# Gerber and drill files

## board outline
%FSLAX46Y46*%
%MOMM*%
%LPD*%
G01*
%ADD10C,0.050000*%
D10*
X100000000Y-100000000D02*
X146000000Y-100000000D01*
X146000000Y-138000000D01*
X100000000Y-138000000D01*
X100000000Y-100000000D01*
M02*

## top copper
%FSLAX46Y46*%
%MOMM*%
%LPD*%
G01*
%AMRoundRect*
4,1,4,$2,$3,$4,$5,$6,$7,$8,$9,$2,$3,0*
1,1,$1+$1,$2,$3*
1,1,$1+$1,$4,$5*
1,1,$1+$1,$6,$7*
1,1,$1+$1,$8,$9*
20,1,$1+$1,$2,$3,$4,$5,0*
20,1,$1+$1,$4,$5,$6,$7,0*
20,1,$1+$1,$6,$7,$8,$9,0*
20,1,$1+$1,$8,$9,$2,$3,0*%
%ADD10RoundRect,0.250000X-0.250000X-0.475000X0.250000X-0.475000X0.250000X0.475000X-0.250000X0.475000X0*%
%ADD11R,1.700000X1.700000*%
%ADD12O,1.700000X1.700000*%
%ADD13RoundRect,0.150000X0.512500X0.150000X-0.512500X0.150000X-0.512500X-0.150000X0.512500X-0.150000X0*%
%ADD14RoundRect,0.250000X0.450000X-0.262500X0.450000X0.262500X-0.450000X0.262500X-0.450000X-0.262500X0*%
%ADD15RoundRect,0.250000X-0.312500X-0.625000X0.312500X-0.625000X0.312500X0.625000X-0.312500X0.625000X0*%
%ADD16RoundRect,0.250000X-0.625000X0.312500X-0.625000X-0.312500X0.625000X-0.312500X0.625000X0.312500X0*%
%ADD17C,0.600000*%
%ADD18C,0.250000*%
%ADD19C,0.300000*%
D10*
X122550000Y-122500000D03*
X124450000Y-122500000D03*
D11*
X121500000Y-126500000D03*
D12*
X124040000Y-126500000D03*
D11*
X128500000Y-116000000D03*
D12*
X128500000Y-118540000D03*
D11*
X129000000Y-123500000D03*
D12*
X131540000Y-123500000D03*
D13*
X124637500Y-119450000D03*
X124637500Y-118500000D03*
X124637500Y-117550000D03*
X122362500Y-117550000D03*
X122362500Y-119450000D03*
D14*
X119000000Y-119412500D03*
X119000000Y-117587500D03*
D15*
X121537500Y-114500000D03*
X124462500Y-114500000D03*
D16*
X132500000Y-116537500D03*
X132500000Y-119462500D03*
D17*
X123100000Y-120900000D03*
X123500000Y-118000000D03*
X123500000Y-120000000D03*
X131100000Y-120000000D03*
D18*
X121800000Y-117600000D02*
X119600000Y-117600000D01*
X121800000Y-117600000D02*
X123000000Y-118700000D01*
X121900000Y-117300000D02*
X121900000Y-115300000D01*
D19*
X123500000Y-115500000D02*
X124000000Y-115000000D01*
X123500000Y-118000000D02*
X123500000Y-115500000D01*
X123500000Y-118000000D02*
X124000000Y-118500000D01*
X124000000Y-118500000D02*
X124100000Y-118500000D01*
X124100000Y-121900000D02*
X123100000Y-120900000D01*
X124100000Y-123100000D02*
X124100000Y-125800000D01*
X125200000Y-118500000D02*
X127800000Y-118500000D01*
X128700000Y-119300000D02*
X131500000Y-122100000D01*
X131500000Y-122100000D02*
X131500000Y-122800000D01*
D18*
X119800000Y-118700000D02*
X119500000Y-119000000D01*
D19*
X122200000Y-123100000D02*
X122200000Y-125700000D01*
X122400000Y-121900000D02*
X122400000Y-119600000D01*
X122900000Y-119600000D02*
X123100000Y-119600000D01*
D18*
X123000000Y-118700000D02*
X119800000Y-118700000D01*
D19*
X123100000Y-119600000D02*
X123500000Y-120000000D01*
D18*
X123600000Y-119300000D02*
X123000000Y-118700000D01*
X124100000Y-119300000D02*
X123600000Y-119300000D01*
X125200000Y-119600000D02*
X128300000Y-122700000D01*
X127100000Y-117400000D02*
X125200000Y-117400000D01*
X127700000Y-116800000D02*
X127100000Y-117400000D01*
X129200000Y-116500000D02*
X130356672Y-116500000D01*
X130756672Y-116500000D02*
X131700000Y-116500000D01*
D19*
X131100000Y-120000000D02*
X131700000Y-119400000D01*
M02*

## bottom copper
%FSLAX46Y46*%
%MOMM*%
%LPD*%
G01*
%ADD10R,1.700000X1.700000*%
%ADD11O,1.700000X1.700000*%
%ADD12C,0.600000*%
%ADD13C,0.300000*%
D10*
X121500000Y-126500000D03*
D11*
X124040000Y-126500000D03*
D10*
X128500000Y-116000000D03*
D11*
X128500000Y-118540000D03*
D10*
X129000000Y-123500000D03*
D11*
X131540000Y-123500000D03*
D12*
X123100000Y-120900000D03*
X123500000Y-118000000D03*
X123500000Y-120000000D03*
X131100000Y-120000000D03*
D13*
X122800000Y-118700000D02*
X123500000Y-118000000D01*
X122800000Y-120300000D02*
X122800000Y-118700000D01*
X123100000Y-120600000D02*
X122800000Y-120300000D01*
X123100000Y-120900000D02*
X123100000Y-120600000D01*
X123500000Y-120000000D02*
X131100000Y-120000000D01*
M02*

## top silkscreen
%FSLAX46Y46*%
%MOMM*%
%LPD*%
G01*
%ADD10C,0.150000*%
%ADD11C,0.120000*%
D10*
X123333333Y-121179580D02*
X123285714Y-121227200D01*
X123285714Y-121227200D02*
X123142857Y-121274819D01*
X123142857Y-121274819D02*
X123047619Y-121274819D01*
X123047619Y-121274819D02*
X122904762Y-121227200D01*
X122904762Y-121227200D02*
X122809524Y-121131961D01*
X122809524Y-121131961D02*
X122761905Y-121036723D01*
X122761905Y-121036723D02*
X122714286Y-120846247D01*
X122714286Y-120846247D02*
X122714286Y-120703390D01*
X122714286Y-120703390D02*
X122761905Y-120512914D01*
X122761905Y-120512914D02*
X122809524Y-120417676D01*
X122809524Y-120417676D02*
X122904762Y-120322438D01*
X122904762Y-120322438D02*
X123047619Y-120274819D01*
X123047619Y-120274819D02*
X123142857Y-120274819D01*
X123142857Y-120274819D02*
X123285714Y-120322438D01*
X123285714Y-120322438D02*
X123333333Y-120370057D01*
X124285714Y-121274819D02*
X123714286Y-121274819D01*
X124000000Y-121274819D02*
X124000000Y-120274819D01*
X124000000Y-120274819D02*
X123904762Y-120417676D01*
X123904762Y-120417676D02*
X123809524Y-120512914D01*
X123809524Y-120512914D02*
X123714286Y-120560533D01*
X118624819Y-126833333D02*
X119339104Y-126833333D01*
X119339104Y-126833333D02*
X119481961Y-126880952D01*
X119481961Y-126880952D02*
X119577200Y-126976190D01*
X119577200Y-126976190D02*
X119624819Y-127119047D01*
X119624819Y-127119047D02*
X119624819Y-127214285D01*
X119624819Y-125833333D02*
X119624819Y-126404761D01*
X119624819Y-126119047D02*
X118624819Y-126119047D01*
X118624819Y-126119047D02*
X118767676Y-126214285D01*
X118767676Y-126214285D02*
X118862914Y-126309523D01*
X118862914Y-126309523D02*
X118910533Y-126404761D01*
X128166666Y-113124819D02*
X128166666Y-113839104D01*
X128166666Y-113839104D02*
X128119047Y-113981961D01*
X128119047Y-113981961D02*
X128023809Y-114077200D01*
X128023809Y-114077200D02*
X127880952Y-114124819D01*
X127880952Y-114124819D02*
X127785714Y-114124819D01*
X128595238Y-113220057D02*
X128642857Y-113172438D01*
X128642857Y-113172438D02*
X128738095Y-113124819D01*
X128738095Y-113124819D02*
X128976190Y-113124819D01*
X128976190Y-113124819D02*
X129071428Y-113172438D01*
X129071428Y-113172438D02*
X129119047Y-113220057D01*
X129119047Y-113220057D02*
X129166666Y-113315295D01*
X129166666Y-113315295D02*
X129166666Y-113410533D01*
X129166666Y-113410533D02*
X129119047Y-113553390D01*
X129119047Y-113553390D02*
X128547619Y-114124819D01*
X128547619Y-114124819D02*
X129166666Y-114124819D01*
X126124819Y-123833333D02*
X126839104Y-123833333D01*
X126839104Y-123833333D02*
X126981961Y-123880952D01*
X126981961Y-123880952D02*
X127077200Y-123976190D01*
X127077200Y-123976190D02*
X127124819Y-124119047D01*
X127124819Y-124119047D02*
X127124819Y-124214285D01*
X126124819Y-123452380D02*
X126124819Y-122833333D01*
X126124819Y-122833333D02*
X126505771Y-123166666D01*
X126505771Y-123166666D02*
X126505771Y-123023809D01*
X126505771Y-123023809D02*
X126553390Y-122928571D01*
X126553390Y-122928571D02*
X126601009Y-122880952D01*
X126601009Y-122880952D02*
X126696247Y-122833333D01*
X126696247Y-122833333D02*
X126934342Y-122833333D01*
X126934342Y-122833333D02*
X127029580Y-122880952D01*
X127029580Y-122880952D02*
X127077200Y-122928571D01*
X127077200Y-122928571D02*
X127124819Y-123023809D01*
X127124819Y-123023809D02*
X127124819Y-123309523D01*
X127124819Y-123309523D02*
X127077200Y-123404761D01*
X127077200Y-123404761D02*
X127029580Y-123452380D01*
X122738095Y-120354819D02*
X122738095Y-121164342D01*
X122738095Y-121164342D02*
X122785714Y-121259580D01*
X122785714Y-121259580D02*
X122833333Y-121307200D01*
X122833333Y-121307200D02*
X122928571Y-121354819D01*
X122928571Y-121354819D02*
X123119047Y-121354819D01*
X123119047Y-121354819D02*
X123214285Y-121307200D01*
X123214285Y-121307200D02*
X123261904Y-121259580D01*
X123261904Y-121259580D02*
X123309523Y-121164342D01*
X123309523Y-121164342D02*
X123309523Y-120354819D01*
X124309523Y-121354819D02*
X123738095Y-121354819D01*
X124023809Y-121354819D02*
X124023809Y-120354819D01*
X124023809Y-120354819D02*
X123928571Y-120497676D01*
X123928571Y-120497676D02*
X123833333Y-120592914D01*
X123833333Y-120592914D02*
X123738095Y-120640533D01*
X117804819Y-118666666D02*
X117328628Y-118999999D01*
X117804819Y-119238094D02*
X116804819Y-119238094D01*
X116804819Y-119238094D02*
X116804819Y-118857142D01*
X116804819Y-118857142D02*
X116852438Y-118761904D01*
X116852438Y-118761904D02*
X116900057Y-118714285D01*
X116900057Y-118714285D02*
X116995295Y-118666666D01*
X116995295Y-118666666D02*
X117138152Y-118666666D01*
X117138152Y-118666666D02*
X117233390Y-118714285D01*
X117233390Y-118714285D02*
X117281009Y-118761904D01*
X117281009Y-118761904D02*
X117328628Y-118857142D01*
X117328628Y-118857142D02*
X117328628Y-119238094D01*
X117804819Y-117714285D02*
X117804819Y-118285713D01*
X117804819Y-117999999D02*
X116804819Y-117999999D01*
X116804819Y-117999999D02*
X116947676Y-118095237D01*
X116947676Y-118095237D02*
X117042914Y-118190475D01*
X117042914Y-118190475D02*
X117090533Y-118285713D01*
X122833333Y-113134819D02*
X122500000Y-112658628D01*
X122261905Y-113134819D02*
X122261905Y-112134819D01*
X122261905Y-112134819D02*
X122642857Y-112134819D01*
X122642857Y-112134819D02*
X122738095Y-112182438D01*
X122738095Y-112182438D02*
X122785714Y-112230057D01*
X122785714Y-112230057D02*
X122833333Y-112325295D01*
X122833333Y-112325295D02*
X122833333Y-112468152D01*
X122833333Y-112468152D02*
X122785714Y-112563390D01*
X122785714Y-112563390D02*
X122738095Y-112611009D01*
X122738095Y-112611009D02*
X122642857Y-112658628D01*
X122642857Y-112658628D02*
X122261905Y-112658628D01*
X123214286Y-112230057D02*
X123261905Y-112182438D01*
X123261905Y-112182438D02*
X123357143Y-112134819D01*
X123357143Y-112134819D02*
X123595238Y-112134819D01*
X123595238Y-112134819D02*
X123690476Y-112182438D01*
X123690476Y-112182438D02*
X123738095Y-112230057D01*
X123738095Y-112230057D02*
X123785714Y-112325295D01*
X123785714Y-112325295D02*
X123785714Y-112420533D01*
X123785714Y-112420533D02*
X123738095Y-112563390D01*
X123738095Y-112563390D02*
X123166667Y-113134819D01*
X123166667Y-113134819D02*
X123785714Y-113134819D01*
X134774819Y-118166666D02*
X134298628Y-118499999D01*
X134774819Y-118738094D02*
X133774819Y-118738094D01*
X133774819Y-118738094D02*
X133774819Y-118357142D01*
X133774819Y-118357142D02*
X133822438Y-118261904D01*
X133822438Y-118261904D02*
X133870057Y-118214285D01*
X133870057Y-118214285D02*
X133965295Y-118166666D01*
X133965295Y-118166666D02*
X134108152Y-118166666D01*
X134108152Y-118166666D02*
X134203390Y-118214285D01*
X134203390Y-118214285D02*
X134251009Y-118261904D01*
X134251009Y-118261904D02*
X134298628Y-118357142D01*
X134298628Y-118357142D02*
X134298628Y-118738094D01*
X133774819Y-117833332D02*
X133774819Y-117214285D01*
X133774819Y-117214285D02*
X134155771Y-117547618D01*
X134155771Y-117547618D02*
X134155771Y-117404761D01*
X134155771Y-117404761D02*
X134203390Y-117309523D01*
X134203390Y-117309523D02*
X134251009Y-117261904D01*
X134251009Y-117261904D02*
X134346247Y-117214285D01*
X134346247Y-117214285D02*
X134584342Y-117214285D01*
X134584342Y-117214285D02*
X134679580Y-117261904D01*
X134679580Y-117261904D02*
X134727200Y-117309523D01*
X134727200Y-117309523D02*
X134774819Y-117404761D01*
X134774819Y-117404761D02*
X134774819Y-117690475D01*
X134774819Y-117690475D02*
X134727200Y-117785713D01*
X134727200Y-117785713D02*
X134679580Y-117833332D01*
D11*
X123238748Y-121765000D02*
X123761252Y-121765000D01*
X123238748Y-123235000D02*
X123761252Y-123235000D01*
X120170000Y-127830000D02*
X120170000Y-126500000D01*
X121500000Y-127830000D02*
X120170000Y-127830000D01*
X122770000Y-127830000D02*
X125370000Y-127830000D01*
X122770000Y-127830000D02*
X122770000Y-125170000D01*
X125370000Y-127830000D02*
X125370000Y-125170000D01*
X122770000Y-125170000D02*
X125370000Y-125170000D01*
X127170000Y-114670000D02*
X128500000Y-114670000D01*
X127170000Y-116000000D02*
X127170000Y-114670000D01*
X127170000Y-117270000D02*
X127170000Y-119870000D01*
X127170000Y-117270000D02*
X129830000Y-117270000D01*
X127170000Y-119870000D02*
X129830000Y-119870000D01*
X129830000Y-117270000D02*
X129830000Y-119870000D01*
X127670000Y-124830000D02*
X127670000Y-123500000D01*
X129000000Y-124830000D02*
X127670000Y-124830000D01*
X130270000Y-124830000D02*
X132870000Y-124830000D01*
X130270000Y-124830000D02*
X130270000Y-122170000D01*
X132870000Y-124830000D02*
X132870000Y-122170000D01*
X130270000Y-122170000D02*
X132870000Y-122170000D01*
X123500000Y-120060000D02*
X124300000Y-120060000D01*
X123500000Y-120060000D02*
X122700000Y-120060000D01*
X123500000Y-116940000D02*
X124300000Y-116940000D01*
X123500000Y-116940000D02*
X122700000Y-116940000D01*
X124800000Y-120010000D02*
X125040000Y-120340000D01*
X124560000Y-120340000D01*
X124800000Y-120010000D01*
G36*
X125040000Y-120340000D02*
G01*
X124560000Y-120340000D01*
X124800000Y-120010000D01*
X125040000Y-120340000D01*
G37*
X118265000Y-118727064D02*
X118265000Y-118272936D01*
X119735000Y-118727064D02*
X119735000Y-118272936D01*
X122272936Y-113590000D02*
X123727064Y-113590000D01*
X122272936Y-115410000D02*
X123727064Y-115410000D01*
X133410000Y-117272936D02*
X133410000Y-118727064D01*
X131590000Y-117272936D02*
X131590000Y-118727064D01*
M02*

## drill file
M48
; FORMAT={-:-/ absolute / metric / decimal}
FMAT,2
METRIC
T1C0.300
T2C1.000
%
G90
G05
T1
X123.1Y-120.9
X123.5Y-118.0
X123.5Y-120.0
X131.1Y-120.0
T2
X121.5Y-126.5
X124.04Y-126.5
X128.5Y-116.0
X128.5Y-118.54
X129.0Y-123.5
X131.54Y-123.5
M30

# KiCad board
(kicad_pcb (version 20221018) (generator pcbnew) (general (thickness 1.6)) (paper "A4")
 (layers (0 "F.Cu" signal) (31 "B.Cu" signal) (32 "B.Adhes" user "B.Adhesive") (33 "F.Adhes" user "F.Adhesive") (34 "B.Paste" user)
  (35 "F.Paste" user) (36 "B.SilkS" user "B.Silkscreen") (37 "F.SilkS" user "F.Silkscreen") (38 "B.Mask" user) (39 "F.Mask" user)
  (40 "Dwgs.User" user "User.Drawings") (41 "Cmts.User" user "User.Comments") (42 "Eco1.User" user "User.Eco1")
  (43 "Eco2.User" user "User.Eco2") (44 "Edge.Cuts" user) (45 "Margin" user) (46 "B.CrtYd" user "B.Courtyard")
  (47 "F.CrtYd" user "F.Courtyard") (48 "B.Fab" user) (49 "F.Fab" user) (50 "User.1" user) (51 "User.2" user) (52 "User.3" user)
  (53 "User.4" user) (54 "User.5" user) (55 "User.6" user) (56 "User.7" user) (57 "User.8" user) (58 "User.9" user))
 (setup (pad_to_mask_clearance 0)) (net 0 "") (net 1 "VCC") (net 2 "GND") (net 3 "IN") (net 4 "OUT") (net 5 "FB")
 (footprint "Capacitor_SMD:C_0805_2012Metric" (layer "F.Cu") (at 123.5 122.5)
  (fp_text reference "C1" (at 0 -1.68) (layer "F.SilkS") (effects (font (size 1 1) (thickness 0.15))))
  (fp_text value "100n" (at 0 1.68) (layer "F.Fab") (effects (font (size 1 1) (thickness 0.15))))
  (fp_line (start -0.261252 -0.735) (end 0.261252 -0.735) (stroke (width 0.12) (type solid)) (layer "F.SilkS"))
  (fp_line (start -0.261252 0.735) (end 0.261252 0.735) (stroke (width 0.12) (type solid)) (layer "F.SilkS"))
  (pad "1" smd roundrect (at -0.95 0) (size 1 1.45) (layers "F.Cu" "F.Paste" "F.Mask") (roundrect_rratio 0.25) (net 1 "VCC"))
  (pad "2" smd roundrect (at 0.95 0) (size 1 1.45) (layers "F.Cu" "F.Paste" "F.Mask") (roundrect_rratio 0.25) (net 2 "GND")))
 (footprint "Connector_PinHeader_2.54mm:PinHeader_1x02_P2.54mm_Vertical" (layer "F.Cu") (at 121.5 126.5 90)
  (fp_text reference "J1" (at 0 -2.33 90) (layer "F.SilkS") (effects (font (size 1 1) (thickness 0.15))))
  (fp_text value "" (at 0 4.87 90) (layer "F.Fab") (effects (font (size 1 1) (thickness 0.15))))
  (fp_line (start -1.33 -1.33) (end 0 -1.33) (stroke (width 0.12) (type solid)) (layer "F.SilkS"))
  (fp_line (start -1.33 0) (end -1.33 -1.33) (stroke (width 0.12) (type solid)) (layer "F.SilkS"))
  (fp_line (start -1.33 1.27) (end -1.33 3.87) (stroke (width 0.12) (type solid)) (layer "F.SilkS"))
  (fp_line (start -1.33 1.27) (end 1.33 1.27) (stroke (width 0.12) (type solid)) (layer "F.SilkS"))
  (fp_line (start -1.33 3.87) (end 1.33 3.87) (stroke (width 0.12) (type solid)) (layer "F.SilkS"))
  (fp_line (start 1.33 1.27) (end 1.33 3.87) (stroke (width 0.12) (type solid)) (layer "F.SilkS"))
  (pad "1" thru_hole rect (at 0 0 90) (size 1.7 1.7) (drill 1) (layers "*.Cu" "*.Mask") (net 1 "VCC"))
  (pad "2" thru_hole oval (at 0 2.54 90) (size 1.7 1.7) (drill 1) (layers "*.Cu" "*.Mask") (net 2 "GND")))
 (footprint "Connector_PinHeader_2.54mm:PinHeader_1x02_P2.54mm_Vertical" (layer "F.Cu") (at 128.5 116)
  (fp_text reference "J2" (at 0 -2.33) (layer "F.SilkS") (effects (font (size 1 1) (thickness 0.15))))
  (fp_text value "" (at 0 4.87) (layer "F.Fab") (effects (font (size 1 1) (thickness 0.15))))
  (fp_line (start -1.33 -1.33) (end 0 -1.33) (stroke (width 0.12) (type solid)) (layer "F.SilkS"))
  (fp_line (start -1.33 0) (end -1.33 -1.33) (stroke (width 0.12) (type solid)) (layer "F.SilkS"))
  (fp_line (start -1.33 1.27) (end -1.33 3.87) (stroke (width 0.12) (type solid)) (layer "F.SilkS"))
  (fp_line (start -1.33 1.27) (end 1.33 1.27) (stroke (width 0.12) (type solid)) (layer "F.SilkS"))
  (fp_line (start -1.33 3.87) (end 1.33 3.87) (stroke (width 0.12) (type solid)) (layer "F.SilkS"))
  (fp_line (start 1.33 1.27) (end 1.33 3.87) (stroke (width 0.12) (type solid)) (layer "F.SilkS"))
  (pad "1" thru_hole rect (at 0 0) (size 1.7 1.7) (drill 1) (layers "*.Cu" "*.Mask") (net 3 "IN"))
  (pad "2" thru_hole oval (at 0 2.54) (size 1.7 1.7) (drill 1) (layers "*.Cu" "*.Mask") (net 2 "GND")))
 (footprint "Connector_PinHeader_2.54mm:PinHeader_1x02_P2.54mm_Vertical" (layer "F.Cu") (at 129 123.5 90)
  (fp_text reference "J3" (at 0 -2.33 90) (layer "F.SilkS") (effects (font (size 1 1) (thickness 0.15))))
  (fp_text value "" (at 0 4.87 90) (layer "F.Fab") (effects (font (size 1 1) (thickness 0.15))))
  (fp_line (start -1.33 -1.33) (end 0 -1.33) (stroke (width 0.12) (type solid)) (layer "F.SilkS"))
  (fp_line (start -1.33 0) (end -1.33 -1.33) (stroke (width 0.12) (type solid)) (layer "F.SilkS"))
  (fp_line (start -1.33 1.27) (end -1.33 3.87) (stroke (width 0.12) (type solid)) (layer "F.SilkS"))
  (fp_line (start -1.33 1.27) (end 1.33 1.27) (stroke (width 0.12) (type solid)) (layer "F.SilkS"))
  (fp_line (start -1.33 3.87) (end 1.33 3.87) (stroke (width 0.12) (type solid)) (layer "F.SilkS"))
  (fp_line (start 1.33 1.27) (end 1.33 3.87) (stroke (width 0.12) (type solid)) (layer "F.SilkS"))
  (pad "1" thru_hole rect (at 0 0 90) (size 1.7 1.7) (drill 1) (layers "*.Cu" "*.Mask") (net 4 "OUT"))
  (pad "2" thru_hole oval (at 0 2.54 90) (size 1.7 1.7) (drill 1) (layers "*.Cu" "*.Mask") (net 2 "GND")))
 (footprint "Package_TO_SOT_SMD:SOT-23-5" (layer "F.Cu") (at 123.5 118.5 180)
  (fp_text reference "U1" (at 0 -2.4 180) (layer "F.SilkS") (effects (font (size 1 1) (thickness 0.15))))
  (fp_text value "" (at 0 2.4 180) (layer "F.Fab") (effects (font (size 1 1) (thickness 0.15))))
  (fp_line (start 0 -1.56) (end -0.8 -1.56) (stroke (width 0.12) (type solid)) (layer "F.SilkS"))
  (fp_line (start 0 -1.56) (end 0.8 -1.56) (stroke (width 0.12) (type solid)) (layer "F.SilkS"))
  (fp_line (start 0 1.56) (end -0.8 1.56) (stroke (width 0.12) (type solid)) (layer "F.SilkS"))
  (fp_line (start 0 1.56) (end 0.8 1.56) (stroke (width 0.12) (type solid)) (layer "F.SilkS"))
  (fp_poly
   (pts (xy -1.3 -1.51) (xy -1.54 -1.84) (xy -1.06 -1.84) (xy -1.3 -1.51)) (stroke (width 0.12) (type solid)) (fill solid) (layer "F.SilkS"))
  (pad "1" smd roundrect (at -1.1375 -0.95 180) (size 1.325 0.6) (layers "F.Cu" "F.Paste" "F.Mask") (roundrect_rratio 0.25) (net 4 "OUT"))
  (pad "2" smd roundrect (at -1.1375 0 180) (size 1.325 0.6) (layers "F.Cu" "F.Paste" "F.Mask") (roundrect_rratio 0.25) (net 2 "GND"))
  (pad "3" smd roundrect (at -1.1375 0.95 180) (size 1.325 0.6) (layers "F.Cu" "F.Paste" "F.Mask") (roundrect_rratio 0.25) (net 3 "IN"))
  (pad "4" smd roundrect (at 1.1375 0.95 180) (size 1.325 0.6) (layers "F.Cu" "F.Paste" "F.Mask") (roundrect_rratio 0.25) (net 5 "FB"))
  (pad "5" smd roundrect (at 1.1375 -0.95 180) (size 1.325 0.6) (layers "F.Cu" "F.Paste" "F.Mask") (roundrect_rratio 0.25) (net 1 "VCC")))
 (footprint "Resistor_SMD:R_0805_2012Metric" (layer "F.Cu") (at 119 118.5 90)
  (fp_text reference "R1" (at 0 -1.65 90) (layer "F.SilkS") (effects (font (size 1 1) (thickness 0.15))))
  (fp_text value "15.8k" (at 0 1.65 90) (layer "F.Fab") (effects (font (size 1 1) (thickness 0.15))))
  (fp_line (start -0.227064 -0.735) (end 0.227064 -0.735) (stroke (width 0.12) (type solid)) (layer "F.SilkS"))
  (fp_line (start -0.227064 0.735) (end 0.227064 0.735) (stroke (width 0.12) (type solid)) (layer "F.SilkS"))
  (pad "1" smd roundrect (at -0.9125 0 90) (size 1.025 1.4) (layers "F.Cu" "F.Paste" "F.Mask") (roundrect_rratio 0.243902) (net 4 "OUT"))
  (pad "2" smd roundrect (at 0.9125 0 90) (size 1.025 1.4) (layers "F.Cu" "F.Paste" "F.Mask") (roundrect_rratio 0.243902) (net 5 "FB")))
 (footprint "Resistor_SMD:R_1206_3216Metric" (layer "F.Cu") (at 123 114.5)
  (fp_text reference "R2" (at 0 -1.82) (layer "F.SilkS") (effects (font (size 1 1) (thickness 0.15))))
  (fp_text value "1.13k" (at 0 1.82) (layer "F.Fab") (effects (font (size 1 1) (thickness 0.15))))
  (fp_line (start -0.727064 -0.91) (end 0.727064 -0.91) (stroke (width 0.12) (type solid)) (layer "F.SilkS"))
  (fp_line (start -0.727064 0.91) (end 0.727064 0.91) (stroke (width 0.12) (type solid)) (layer "F.SilkS"))
  (pad "1" smd roundrect (at -1.4625 0) (size 1.125 1.75) (layers "F.Cu" "F.Paste" "F.Mask") (roundrect_rratio 0.222222) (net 5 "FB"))
  (pad "2" smd roundrect (at 1.4625 0) (size 1.125 1.75) (layers "F.Cu" "F.Paste" "F.Mask") (roundrect_rratio 0.222222) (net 2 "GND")))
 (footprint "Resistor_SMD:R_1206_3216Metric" (layer "F.Cu") (at 132.5 118 -90)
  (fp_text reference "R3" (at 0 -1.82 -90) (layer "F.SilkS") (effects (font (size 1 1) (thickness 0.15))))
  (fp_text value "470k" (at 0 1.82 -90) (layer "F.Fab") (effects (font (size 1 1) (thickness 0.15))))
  (fp_line (start -0.727064 -0.91) (end 0.727064 -0.91) (stroke (width 0.12) (type solid)) (layer "F.SilkS"))
  (fp_line (start -0.727064 0.91) (end 0.727064 0.91) (stroke (width 0.12) (type solid)) (layer "F.SilkS"))
  (pad "1" smd roundrect (at -1.4625 0 270) (size 1.125 1.75) (layers "F.Cu" "F.Paste" "F.Mask") (roundrect_rratio 0.222222) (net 3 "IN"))
  (pad "2" smd roundrect (at 1.4625 0 270) (size 1.125 1.75) (layers "F.Cu" "F.Paste" "F.Mask") (roundrect_rratio 0.222222) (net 1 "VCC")))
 (gr_rect (start 100 100) (end 146 138) (stroke (width 0.05) (type default)) (fill none) (layer "Edge.Cuts"))
 (segment (start 121.8 117.6) (end 119.6 117.6) (width 0.25) (layer "F.Cu") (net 5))
 (segment (start 121.8 117.6) (end 123 118.7) (width 0.25) (layer "F.Cu") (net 5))
 (segment (start 121.9 117.3) (end 121.9 115.3) (width 0.25) (layer "F.Cu") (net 5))
 (segment (start 123.5 115.5) (end 124 115) (width 0.3) (layer "F.Cu") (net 2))
 (segment (start 123.5 118) (end 123.5 115.5) (width 0.3) (layer "F.Cu") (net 2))
 (segment (start 123.5 118) (end 124 118.5) (width 0.3) (layer "F.Cu") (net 2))
 (segment (start 124 118.5) (end 124.1 118.5) (width 0.3) (layer "F.Cu") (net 2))
 (segment (start 124.1 121.9) (end 123.1 120.9) (width 0.3) (layer "F.Cu") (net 2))
 (segment (start 124.1 123.1) (end 124.1 125.8) (width 0.3) (layer "F.Cu") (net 2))
 (segment (start 125.2 118.5) (end 127.8 118.5) (width 0.3) (layer "F.Cu") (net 2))
 (segment (start 128.7 119.3) (end 131.5 122.1) (width 0.3) (layer "F.Cu") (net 2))
 (segment (start 131.5 122.1) (end 131.5 122.8) (width 0.3) (layer "F.Cu") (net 2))
 (via (at 123.1 120.9) (size 0.6) (drill 0.3) (layers "F.Cu" "B.Cu") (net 2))
 (via (at 123.5 118) (size 0.6) (drill 0.3) (layers "F.Cu" "B.Cu") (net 2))
 (segment (start 119.8 118.7) (end 119.5 119) (width 0.25) (layer "F.Cu") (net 4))
 (segment (start 122.2 123.1) (end 122.2 125.7) (width 0.3) (layer "F.Cu") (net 1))
 (segment (start 122.4 121.9) (end 122.4 119.6) (width 0.3) (layer "F.Cu") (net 1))
 (segment (start 122.8 118.7) (end 123.5 118) (width 0.3) (layer "B.Cu") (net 2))
 (segment (start 122.8 120.3) (end 122.8 118.7) (width 0.3) (layer "B.Cu") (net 2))
 (segment (start 122.9 119.6) (end 123.1 119.6) (width 0.3) (layer "F.Cu") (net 1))
 (segment (start 123 118.7) (end 119.8 118.7) (width 0.25) (layer "F.Cu") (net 4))
 (segment (start 123.1 119.6) (end 123.5 120) (width 0.3) (layer "F.Cu") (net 1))
 (segment (start 123.1 120.6) (end 122.8 120.3) (width 0.3) (layer "B.Cu") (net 2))
 (segment (start 123.1 120.9) (end 123.1 120.6) (width 0.3) (layer "B.Cu") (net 2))
 (segment (start 123.6 119.3) (end 123 118.7) (width 0.25) (layer "F.Cu") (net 4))
 (segment (start 124.1 119.3) (end 123.6 119.3) (width 0.25) (layer "F.Cu") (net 4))
 (segment (start 125.2 119.6) (end 128.3 122.7) (width 0.25) (layer "F.Cu") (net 4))
 (segment (start 127.1 117.4) (end 125.2 117.4) (width 0.25) (layer "F.Cu") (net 3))
 (segment (start 127.7 116.8) (end 127.1 117.4) (width 0.25) (layer "F.Cu") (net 3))
 (segment (start 129.2 116.5) (end 130.356672 116.5) (width 0.25) (layer "F.Cu") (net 3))
 (segment (start 130.756672 116.5) (end 131.7 116.5) (width 0.25) (layer "F.Cu") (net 3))
 (segment (start 131.1 120) (end 131.7 119.4) (width 0.3) (layer "F.Cu") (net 1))
 (via (at 123.5 120) (size 0.6) (drill 0.3) (layers "F.Cu" "B.Cu") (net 1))
 (via (at 131.1 120) (size 0.6) (drill 0.3) (layers "F.Cu" "B.Cu") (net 1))
 (segment (start 123.5 120) (end 131.1 120) (width 0.3) (layer "B.Cu") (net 1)))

